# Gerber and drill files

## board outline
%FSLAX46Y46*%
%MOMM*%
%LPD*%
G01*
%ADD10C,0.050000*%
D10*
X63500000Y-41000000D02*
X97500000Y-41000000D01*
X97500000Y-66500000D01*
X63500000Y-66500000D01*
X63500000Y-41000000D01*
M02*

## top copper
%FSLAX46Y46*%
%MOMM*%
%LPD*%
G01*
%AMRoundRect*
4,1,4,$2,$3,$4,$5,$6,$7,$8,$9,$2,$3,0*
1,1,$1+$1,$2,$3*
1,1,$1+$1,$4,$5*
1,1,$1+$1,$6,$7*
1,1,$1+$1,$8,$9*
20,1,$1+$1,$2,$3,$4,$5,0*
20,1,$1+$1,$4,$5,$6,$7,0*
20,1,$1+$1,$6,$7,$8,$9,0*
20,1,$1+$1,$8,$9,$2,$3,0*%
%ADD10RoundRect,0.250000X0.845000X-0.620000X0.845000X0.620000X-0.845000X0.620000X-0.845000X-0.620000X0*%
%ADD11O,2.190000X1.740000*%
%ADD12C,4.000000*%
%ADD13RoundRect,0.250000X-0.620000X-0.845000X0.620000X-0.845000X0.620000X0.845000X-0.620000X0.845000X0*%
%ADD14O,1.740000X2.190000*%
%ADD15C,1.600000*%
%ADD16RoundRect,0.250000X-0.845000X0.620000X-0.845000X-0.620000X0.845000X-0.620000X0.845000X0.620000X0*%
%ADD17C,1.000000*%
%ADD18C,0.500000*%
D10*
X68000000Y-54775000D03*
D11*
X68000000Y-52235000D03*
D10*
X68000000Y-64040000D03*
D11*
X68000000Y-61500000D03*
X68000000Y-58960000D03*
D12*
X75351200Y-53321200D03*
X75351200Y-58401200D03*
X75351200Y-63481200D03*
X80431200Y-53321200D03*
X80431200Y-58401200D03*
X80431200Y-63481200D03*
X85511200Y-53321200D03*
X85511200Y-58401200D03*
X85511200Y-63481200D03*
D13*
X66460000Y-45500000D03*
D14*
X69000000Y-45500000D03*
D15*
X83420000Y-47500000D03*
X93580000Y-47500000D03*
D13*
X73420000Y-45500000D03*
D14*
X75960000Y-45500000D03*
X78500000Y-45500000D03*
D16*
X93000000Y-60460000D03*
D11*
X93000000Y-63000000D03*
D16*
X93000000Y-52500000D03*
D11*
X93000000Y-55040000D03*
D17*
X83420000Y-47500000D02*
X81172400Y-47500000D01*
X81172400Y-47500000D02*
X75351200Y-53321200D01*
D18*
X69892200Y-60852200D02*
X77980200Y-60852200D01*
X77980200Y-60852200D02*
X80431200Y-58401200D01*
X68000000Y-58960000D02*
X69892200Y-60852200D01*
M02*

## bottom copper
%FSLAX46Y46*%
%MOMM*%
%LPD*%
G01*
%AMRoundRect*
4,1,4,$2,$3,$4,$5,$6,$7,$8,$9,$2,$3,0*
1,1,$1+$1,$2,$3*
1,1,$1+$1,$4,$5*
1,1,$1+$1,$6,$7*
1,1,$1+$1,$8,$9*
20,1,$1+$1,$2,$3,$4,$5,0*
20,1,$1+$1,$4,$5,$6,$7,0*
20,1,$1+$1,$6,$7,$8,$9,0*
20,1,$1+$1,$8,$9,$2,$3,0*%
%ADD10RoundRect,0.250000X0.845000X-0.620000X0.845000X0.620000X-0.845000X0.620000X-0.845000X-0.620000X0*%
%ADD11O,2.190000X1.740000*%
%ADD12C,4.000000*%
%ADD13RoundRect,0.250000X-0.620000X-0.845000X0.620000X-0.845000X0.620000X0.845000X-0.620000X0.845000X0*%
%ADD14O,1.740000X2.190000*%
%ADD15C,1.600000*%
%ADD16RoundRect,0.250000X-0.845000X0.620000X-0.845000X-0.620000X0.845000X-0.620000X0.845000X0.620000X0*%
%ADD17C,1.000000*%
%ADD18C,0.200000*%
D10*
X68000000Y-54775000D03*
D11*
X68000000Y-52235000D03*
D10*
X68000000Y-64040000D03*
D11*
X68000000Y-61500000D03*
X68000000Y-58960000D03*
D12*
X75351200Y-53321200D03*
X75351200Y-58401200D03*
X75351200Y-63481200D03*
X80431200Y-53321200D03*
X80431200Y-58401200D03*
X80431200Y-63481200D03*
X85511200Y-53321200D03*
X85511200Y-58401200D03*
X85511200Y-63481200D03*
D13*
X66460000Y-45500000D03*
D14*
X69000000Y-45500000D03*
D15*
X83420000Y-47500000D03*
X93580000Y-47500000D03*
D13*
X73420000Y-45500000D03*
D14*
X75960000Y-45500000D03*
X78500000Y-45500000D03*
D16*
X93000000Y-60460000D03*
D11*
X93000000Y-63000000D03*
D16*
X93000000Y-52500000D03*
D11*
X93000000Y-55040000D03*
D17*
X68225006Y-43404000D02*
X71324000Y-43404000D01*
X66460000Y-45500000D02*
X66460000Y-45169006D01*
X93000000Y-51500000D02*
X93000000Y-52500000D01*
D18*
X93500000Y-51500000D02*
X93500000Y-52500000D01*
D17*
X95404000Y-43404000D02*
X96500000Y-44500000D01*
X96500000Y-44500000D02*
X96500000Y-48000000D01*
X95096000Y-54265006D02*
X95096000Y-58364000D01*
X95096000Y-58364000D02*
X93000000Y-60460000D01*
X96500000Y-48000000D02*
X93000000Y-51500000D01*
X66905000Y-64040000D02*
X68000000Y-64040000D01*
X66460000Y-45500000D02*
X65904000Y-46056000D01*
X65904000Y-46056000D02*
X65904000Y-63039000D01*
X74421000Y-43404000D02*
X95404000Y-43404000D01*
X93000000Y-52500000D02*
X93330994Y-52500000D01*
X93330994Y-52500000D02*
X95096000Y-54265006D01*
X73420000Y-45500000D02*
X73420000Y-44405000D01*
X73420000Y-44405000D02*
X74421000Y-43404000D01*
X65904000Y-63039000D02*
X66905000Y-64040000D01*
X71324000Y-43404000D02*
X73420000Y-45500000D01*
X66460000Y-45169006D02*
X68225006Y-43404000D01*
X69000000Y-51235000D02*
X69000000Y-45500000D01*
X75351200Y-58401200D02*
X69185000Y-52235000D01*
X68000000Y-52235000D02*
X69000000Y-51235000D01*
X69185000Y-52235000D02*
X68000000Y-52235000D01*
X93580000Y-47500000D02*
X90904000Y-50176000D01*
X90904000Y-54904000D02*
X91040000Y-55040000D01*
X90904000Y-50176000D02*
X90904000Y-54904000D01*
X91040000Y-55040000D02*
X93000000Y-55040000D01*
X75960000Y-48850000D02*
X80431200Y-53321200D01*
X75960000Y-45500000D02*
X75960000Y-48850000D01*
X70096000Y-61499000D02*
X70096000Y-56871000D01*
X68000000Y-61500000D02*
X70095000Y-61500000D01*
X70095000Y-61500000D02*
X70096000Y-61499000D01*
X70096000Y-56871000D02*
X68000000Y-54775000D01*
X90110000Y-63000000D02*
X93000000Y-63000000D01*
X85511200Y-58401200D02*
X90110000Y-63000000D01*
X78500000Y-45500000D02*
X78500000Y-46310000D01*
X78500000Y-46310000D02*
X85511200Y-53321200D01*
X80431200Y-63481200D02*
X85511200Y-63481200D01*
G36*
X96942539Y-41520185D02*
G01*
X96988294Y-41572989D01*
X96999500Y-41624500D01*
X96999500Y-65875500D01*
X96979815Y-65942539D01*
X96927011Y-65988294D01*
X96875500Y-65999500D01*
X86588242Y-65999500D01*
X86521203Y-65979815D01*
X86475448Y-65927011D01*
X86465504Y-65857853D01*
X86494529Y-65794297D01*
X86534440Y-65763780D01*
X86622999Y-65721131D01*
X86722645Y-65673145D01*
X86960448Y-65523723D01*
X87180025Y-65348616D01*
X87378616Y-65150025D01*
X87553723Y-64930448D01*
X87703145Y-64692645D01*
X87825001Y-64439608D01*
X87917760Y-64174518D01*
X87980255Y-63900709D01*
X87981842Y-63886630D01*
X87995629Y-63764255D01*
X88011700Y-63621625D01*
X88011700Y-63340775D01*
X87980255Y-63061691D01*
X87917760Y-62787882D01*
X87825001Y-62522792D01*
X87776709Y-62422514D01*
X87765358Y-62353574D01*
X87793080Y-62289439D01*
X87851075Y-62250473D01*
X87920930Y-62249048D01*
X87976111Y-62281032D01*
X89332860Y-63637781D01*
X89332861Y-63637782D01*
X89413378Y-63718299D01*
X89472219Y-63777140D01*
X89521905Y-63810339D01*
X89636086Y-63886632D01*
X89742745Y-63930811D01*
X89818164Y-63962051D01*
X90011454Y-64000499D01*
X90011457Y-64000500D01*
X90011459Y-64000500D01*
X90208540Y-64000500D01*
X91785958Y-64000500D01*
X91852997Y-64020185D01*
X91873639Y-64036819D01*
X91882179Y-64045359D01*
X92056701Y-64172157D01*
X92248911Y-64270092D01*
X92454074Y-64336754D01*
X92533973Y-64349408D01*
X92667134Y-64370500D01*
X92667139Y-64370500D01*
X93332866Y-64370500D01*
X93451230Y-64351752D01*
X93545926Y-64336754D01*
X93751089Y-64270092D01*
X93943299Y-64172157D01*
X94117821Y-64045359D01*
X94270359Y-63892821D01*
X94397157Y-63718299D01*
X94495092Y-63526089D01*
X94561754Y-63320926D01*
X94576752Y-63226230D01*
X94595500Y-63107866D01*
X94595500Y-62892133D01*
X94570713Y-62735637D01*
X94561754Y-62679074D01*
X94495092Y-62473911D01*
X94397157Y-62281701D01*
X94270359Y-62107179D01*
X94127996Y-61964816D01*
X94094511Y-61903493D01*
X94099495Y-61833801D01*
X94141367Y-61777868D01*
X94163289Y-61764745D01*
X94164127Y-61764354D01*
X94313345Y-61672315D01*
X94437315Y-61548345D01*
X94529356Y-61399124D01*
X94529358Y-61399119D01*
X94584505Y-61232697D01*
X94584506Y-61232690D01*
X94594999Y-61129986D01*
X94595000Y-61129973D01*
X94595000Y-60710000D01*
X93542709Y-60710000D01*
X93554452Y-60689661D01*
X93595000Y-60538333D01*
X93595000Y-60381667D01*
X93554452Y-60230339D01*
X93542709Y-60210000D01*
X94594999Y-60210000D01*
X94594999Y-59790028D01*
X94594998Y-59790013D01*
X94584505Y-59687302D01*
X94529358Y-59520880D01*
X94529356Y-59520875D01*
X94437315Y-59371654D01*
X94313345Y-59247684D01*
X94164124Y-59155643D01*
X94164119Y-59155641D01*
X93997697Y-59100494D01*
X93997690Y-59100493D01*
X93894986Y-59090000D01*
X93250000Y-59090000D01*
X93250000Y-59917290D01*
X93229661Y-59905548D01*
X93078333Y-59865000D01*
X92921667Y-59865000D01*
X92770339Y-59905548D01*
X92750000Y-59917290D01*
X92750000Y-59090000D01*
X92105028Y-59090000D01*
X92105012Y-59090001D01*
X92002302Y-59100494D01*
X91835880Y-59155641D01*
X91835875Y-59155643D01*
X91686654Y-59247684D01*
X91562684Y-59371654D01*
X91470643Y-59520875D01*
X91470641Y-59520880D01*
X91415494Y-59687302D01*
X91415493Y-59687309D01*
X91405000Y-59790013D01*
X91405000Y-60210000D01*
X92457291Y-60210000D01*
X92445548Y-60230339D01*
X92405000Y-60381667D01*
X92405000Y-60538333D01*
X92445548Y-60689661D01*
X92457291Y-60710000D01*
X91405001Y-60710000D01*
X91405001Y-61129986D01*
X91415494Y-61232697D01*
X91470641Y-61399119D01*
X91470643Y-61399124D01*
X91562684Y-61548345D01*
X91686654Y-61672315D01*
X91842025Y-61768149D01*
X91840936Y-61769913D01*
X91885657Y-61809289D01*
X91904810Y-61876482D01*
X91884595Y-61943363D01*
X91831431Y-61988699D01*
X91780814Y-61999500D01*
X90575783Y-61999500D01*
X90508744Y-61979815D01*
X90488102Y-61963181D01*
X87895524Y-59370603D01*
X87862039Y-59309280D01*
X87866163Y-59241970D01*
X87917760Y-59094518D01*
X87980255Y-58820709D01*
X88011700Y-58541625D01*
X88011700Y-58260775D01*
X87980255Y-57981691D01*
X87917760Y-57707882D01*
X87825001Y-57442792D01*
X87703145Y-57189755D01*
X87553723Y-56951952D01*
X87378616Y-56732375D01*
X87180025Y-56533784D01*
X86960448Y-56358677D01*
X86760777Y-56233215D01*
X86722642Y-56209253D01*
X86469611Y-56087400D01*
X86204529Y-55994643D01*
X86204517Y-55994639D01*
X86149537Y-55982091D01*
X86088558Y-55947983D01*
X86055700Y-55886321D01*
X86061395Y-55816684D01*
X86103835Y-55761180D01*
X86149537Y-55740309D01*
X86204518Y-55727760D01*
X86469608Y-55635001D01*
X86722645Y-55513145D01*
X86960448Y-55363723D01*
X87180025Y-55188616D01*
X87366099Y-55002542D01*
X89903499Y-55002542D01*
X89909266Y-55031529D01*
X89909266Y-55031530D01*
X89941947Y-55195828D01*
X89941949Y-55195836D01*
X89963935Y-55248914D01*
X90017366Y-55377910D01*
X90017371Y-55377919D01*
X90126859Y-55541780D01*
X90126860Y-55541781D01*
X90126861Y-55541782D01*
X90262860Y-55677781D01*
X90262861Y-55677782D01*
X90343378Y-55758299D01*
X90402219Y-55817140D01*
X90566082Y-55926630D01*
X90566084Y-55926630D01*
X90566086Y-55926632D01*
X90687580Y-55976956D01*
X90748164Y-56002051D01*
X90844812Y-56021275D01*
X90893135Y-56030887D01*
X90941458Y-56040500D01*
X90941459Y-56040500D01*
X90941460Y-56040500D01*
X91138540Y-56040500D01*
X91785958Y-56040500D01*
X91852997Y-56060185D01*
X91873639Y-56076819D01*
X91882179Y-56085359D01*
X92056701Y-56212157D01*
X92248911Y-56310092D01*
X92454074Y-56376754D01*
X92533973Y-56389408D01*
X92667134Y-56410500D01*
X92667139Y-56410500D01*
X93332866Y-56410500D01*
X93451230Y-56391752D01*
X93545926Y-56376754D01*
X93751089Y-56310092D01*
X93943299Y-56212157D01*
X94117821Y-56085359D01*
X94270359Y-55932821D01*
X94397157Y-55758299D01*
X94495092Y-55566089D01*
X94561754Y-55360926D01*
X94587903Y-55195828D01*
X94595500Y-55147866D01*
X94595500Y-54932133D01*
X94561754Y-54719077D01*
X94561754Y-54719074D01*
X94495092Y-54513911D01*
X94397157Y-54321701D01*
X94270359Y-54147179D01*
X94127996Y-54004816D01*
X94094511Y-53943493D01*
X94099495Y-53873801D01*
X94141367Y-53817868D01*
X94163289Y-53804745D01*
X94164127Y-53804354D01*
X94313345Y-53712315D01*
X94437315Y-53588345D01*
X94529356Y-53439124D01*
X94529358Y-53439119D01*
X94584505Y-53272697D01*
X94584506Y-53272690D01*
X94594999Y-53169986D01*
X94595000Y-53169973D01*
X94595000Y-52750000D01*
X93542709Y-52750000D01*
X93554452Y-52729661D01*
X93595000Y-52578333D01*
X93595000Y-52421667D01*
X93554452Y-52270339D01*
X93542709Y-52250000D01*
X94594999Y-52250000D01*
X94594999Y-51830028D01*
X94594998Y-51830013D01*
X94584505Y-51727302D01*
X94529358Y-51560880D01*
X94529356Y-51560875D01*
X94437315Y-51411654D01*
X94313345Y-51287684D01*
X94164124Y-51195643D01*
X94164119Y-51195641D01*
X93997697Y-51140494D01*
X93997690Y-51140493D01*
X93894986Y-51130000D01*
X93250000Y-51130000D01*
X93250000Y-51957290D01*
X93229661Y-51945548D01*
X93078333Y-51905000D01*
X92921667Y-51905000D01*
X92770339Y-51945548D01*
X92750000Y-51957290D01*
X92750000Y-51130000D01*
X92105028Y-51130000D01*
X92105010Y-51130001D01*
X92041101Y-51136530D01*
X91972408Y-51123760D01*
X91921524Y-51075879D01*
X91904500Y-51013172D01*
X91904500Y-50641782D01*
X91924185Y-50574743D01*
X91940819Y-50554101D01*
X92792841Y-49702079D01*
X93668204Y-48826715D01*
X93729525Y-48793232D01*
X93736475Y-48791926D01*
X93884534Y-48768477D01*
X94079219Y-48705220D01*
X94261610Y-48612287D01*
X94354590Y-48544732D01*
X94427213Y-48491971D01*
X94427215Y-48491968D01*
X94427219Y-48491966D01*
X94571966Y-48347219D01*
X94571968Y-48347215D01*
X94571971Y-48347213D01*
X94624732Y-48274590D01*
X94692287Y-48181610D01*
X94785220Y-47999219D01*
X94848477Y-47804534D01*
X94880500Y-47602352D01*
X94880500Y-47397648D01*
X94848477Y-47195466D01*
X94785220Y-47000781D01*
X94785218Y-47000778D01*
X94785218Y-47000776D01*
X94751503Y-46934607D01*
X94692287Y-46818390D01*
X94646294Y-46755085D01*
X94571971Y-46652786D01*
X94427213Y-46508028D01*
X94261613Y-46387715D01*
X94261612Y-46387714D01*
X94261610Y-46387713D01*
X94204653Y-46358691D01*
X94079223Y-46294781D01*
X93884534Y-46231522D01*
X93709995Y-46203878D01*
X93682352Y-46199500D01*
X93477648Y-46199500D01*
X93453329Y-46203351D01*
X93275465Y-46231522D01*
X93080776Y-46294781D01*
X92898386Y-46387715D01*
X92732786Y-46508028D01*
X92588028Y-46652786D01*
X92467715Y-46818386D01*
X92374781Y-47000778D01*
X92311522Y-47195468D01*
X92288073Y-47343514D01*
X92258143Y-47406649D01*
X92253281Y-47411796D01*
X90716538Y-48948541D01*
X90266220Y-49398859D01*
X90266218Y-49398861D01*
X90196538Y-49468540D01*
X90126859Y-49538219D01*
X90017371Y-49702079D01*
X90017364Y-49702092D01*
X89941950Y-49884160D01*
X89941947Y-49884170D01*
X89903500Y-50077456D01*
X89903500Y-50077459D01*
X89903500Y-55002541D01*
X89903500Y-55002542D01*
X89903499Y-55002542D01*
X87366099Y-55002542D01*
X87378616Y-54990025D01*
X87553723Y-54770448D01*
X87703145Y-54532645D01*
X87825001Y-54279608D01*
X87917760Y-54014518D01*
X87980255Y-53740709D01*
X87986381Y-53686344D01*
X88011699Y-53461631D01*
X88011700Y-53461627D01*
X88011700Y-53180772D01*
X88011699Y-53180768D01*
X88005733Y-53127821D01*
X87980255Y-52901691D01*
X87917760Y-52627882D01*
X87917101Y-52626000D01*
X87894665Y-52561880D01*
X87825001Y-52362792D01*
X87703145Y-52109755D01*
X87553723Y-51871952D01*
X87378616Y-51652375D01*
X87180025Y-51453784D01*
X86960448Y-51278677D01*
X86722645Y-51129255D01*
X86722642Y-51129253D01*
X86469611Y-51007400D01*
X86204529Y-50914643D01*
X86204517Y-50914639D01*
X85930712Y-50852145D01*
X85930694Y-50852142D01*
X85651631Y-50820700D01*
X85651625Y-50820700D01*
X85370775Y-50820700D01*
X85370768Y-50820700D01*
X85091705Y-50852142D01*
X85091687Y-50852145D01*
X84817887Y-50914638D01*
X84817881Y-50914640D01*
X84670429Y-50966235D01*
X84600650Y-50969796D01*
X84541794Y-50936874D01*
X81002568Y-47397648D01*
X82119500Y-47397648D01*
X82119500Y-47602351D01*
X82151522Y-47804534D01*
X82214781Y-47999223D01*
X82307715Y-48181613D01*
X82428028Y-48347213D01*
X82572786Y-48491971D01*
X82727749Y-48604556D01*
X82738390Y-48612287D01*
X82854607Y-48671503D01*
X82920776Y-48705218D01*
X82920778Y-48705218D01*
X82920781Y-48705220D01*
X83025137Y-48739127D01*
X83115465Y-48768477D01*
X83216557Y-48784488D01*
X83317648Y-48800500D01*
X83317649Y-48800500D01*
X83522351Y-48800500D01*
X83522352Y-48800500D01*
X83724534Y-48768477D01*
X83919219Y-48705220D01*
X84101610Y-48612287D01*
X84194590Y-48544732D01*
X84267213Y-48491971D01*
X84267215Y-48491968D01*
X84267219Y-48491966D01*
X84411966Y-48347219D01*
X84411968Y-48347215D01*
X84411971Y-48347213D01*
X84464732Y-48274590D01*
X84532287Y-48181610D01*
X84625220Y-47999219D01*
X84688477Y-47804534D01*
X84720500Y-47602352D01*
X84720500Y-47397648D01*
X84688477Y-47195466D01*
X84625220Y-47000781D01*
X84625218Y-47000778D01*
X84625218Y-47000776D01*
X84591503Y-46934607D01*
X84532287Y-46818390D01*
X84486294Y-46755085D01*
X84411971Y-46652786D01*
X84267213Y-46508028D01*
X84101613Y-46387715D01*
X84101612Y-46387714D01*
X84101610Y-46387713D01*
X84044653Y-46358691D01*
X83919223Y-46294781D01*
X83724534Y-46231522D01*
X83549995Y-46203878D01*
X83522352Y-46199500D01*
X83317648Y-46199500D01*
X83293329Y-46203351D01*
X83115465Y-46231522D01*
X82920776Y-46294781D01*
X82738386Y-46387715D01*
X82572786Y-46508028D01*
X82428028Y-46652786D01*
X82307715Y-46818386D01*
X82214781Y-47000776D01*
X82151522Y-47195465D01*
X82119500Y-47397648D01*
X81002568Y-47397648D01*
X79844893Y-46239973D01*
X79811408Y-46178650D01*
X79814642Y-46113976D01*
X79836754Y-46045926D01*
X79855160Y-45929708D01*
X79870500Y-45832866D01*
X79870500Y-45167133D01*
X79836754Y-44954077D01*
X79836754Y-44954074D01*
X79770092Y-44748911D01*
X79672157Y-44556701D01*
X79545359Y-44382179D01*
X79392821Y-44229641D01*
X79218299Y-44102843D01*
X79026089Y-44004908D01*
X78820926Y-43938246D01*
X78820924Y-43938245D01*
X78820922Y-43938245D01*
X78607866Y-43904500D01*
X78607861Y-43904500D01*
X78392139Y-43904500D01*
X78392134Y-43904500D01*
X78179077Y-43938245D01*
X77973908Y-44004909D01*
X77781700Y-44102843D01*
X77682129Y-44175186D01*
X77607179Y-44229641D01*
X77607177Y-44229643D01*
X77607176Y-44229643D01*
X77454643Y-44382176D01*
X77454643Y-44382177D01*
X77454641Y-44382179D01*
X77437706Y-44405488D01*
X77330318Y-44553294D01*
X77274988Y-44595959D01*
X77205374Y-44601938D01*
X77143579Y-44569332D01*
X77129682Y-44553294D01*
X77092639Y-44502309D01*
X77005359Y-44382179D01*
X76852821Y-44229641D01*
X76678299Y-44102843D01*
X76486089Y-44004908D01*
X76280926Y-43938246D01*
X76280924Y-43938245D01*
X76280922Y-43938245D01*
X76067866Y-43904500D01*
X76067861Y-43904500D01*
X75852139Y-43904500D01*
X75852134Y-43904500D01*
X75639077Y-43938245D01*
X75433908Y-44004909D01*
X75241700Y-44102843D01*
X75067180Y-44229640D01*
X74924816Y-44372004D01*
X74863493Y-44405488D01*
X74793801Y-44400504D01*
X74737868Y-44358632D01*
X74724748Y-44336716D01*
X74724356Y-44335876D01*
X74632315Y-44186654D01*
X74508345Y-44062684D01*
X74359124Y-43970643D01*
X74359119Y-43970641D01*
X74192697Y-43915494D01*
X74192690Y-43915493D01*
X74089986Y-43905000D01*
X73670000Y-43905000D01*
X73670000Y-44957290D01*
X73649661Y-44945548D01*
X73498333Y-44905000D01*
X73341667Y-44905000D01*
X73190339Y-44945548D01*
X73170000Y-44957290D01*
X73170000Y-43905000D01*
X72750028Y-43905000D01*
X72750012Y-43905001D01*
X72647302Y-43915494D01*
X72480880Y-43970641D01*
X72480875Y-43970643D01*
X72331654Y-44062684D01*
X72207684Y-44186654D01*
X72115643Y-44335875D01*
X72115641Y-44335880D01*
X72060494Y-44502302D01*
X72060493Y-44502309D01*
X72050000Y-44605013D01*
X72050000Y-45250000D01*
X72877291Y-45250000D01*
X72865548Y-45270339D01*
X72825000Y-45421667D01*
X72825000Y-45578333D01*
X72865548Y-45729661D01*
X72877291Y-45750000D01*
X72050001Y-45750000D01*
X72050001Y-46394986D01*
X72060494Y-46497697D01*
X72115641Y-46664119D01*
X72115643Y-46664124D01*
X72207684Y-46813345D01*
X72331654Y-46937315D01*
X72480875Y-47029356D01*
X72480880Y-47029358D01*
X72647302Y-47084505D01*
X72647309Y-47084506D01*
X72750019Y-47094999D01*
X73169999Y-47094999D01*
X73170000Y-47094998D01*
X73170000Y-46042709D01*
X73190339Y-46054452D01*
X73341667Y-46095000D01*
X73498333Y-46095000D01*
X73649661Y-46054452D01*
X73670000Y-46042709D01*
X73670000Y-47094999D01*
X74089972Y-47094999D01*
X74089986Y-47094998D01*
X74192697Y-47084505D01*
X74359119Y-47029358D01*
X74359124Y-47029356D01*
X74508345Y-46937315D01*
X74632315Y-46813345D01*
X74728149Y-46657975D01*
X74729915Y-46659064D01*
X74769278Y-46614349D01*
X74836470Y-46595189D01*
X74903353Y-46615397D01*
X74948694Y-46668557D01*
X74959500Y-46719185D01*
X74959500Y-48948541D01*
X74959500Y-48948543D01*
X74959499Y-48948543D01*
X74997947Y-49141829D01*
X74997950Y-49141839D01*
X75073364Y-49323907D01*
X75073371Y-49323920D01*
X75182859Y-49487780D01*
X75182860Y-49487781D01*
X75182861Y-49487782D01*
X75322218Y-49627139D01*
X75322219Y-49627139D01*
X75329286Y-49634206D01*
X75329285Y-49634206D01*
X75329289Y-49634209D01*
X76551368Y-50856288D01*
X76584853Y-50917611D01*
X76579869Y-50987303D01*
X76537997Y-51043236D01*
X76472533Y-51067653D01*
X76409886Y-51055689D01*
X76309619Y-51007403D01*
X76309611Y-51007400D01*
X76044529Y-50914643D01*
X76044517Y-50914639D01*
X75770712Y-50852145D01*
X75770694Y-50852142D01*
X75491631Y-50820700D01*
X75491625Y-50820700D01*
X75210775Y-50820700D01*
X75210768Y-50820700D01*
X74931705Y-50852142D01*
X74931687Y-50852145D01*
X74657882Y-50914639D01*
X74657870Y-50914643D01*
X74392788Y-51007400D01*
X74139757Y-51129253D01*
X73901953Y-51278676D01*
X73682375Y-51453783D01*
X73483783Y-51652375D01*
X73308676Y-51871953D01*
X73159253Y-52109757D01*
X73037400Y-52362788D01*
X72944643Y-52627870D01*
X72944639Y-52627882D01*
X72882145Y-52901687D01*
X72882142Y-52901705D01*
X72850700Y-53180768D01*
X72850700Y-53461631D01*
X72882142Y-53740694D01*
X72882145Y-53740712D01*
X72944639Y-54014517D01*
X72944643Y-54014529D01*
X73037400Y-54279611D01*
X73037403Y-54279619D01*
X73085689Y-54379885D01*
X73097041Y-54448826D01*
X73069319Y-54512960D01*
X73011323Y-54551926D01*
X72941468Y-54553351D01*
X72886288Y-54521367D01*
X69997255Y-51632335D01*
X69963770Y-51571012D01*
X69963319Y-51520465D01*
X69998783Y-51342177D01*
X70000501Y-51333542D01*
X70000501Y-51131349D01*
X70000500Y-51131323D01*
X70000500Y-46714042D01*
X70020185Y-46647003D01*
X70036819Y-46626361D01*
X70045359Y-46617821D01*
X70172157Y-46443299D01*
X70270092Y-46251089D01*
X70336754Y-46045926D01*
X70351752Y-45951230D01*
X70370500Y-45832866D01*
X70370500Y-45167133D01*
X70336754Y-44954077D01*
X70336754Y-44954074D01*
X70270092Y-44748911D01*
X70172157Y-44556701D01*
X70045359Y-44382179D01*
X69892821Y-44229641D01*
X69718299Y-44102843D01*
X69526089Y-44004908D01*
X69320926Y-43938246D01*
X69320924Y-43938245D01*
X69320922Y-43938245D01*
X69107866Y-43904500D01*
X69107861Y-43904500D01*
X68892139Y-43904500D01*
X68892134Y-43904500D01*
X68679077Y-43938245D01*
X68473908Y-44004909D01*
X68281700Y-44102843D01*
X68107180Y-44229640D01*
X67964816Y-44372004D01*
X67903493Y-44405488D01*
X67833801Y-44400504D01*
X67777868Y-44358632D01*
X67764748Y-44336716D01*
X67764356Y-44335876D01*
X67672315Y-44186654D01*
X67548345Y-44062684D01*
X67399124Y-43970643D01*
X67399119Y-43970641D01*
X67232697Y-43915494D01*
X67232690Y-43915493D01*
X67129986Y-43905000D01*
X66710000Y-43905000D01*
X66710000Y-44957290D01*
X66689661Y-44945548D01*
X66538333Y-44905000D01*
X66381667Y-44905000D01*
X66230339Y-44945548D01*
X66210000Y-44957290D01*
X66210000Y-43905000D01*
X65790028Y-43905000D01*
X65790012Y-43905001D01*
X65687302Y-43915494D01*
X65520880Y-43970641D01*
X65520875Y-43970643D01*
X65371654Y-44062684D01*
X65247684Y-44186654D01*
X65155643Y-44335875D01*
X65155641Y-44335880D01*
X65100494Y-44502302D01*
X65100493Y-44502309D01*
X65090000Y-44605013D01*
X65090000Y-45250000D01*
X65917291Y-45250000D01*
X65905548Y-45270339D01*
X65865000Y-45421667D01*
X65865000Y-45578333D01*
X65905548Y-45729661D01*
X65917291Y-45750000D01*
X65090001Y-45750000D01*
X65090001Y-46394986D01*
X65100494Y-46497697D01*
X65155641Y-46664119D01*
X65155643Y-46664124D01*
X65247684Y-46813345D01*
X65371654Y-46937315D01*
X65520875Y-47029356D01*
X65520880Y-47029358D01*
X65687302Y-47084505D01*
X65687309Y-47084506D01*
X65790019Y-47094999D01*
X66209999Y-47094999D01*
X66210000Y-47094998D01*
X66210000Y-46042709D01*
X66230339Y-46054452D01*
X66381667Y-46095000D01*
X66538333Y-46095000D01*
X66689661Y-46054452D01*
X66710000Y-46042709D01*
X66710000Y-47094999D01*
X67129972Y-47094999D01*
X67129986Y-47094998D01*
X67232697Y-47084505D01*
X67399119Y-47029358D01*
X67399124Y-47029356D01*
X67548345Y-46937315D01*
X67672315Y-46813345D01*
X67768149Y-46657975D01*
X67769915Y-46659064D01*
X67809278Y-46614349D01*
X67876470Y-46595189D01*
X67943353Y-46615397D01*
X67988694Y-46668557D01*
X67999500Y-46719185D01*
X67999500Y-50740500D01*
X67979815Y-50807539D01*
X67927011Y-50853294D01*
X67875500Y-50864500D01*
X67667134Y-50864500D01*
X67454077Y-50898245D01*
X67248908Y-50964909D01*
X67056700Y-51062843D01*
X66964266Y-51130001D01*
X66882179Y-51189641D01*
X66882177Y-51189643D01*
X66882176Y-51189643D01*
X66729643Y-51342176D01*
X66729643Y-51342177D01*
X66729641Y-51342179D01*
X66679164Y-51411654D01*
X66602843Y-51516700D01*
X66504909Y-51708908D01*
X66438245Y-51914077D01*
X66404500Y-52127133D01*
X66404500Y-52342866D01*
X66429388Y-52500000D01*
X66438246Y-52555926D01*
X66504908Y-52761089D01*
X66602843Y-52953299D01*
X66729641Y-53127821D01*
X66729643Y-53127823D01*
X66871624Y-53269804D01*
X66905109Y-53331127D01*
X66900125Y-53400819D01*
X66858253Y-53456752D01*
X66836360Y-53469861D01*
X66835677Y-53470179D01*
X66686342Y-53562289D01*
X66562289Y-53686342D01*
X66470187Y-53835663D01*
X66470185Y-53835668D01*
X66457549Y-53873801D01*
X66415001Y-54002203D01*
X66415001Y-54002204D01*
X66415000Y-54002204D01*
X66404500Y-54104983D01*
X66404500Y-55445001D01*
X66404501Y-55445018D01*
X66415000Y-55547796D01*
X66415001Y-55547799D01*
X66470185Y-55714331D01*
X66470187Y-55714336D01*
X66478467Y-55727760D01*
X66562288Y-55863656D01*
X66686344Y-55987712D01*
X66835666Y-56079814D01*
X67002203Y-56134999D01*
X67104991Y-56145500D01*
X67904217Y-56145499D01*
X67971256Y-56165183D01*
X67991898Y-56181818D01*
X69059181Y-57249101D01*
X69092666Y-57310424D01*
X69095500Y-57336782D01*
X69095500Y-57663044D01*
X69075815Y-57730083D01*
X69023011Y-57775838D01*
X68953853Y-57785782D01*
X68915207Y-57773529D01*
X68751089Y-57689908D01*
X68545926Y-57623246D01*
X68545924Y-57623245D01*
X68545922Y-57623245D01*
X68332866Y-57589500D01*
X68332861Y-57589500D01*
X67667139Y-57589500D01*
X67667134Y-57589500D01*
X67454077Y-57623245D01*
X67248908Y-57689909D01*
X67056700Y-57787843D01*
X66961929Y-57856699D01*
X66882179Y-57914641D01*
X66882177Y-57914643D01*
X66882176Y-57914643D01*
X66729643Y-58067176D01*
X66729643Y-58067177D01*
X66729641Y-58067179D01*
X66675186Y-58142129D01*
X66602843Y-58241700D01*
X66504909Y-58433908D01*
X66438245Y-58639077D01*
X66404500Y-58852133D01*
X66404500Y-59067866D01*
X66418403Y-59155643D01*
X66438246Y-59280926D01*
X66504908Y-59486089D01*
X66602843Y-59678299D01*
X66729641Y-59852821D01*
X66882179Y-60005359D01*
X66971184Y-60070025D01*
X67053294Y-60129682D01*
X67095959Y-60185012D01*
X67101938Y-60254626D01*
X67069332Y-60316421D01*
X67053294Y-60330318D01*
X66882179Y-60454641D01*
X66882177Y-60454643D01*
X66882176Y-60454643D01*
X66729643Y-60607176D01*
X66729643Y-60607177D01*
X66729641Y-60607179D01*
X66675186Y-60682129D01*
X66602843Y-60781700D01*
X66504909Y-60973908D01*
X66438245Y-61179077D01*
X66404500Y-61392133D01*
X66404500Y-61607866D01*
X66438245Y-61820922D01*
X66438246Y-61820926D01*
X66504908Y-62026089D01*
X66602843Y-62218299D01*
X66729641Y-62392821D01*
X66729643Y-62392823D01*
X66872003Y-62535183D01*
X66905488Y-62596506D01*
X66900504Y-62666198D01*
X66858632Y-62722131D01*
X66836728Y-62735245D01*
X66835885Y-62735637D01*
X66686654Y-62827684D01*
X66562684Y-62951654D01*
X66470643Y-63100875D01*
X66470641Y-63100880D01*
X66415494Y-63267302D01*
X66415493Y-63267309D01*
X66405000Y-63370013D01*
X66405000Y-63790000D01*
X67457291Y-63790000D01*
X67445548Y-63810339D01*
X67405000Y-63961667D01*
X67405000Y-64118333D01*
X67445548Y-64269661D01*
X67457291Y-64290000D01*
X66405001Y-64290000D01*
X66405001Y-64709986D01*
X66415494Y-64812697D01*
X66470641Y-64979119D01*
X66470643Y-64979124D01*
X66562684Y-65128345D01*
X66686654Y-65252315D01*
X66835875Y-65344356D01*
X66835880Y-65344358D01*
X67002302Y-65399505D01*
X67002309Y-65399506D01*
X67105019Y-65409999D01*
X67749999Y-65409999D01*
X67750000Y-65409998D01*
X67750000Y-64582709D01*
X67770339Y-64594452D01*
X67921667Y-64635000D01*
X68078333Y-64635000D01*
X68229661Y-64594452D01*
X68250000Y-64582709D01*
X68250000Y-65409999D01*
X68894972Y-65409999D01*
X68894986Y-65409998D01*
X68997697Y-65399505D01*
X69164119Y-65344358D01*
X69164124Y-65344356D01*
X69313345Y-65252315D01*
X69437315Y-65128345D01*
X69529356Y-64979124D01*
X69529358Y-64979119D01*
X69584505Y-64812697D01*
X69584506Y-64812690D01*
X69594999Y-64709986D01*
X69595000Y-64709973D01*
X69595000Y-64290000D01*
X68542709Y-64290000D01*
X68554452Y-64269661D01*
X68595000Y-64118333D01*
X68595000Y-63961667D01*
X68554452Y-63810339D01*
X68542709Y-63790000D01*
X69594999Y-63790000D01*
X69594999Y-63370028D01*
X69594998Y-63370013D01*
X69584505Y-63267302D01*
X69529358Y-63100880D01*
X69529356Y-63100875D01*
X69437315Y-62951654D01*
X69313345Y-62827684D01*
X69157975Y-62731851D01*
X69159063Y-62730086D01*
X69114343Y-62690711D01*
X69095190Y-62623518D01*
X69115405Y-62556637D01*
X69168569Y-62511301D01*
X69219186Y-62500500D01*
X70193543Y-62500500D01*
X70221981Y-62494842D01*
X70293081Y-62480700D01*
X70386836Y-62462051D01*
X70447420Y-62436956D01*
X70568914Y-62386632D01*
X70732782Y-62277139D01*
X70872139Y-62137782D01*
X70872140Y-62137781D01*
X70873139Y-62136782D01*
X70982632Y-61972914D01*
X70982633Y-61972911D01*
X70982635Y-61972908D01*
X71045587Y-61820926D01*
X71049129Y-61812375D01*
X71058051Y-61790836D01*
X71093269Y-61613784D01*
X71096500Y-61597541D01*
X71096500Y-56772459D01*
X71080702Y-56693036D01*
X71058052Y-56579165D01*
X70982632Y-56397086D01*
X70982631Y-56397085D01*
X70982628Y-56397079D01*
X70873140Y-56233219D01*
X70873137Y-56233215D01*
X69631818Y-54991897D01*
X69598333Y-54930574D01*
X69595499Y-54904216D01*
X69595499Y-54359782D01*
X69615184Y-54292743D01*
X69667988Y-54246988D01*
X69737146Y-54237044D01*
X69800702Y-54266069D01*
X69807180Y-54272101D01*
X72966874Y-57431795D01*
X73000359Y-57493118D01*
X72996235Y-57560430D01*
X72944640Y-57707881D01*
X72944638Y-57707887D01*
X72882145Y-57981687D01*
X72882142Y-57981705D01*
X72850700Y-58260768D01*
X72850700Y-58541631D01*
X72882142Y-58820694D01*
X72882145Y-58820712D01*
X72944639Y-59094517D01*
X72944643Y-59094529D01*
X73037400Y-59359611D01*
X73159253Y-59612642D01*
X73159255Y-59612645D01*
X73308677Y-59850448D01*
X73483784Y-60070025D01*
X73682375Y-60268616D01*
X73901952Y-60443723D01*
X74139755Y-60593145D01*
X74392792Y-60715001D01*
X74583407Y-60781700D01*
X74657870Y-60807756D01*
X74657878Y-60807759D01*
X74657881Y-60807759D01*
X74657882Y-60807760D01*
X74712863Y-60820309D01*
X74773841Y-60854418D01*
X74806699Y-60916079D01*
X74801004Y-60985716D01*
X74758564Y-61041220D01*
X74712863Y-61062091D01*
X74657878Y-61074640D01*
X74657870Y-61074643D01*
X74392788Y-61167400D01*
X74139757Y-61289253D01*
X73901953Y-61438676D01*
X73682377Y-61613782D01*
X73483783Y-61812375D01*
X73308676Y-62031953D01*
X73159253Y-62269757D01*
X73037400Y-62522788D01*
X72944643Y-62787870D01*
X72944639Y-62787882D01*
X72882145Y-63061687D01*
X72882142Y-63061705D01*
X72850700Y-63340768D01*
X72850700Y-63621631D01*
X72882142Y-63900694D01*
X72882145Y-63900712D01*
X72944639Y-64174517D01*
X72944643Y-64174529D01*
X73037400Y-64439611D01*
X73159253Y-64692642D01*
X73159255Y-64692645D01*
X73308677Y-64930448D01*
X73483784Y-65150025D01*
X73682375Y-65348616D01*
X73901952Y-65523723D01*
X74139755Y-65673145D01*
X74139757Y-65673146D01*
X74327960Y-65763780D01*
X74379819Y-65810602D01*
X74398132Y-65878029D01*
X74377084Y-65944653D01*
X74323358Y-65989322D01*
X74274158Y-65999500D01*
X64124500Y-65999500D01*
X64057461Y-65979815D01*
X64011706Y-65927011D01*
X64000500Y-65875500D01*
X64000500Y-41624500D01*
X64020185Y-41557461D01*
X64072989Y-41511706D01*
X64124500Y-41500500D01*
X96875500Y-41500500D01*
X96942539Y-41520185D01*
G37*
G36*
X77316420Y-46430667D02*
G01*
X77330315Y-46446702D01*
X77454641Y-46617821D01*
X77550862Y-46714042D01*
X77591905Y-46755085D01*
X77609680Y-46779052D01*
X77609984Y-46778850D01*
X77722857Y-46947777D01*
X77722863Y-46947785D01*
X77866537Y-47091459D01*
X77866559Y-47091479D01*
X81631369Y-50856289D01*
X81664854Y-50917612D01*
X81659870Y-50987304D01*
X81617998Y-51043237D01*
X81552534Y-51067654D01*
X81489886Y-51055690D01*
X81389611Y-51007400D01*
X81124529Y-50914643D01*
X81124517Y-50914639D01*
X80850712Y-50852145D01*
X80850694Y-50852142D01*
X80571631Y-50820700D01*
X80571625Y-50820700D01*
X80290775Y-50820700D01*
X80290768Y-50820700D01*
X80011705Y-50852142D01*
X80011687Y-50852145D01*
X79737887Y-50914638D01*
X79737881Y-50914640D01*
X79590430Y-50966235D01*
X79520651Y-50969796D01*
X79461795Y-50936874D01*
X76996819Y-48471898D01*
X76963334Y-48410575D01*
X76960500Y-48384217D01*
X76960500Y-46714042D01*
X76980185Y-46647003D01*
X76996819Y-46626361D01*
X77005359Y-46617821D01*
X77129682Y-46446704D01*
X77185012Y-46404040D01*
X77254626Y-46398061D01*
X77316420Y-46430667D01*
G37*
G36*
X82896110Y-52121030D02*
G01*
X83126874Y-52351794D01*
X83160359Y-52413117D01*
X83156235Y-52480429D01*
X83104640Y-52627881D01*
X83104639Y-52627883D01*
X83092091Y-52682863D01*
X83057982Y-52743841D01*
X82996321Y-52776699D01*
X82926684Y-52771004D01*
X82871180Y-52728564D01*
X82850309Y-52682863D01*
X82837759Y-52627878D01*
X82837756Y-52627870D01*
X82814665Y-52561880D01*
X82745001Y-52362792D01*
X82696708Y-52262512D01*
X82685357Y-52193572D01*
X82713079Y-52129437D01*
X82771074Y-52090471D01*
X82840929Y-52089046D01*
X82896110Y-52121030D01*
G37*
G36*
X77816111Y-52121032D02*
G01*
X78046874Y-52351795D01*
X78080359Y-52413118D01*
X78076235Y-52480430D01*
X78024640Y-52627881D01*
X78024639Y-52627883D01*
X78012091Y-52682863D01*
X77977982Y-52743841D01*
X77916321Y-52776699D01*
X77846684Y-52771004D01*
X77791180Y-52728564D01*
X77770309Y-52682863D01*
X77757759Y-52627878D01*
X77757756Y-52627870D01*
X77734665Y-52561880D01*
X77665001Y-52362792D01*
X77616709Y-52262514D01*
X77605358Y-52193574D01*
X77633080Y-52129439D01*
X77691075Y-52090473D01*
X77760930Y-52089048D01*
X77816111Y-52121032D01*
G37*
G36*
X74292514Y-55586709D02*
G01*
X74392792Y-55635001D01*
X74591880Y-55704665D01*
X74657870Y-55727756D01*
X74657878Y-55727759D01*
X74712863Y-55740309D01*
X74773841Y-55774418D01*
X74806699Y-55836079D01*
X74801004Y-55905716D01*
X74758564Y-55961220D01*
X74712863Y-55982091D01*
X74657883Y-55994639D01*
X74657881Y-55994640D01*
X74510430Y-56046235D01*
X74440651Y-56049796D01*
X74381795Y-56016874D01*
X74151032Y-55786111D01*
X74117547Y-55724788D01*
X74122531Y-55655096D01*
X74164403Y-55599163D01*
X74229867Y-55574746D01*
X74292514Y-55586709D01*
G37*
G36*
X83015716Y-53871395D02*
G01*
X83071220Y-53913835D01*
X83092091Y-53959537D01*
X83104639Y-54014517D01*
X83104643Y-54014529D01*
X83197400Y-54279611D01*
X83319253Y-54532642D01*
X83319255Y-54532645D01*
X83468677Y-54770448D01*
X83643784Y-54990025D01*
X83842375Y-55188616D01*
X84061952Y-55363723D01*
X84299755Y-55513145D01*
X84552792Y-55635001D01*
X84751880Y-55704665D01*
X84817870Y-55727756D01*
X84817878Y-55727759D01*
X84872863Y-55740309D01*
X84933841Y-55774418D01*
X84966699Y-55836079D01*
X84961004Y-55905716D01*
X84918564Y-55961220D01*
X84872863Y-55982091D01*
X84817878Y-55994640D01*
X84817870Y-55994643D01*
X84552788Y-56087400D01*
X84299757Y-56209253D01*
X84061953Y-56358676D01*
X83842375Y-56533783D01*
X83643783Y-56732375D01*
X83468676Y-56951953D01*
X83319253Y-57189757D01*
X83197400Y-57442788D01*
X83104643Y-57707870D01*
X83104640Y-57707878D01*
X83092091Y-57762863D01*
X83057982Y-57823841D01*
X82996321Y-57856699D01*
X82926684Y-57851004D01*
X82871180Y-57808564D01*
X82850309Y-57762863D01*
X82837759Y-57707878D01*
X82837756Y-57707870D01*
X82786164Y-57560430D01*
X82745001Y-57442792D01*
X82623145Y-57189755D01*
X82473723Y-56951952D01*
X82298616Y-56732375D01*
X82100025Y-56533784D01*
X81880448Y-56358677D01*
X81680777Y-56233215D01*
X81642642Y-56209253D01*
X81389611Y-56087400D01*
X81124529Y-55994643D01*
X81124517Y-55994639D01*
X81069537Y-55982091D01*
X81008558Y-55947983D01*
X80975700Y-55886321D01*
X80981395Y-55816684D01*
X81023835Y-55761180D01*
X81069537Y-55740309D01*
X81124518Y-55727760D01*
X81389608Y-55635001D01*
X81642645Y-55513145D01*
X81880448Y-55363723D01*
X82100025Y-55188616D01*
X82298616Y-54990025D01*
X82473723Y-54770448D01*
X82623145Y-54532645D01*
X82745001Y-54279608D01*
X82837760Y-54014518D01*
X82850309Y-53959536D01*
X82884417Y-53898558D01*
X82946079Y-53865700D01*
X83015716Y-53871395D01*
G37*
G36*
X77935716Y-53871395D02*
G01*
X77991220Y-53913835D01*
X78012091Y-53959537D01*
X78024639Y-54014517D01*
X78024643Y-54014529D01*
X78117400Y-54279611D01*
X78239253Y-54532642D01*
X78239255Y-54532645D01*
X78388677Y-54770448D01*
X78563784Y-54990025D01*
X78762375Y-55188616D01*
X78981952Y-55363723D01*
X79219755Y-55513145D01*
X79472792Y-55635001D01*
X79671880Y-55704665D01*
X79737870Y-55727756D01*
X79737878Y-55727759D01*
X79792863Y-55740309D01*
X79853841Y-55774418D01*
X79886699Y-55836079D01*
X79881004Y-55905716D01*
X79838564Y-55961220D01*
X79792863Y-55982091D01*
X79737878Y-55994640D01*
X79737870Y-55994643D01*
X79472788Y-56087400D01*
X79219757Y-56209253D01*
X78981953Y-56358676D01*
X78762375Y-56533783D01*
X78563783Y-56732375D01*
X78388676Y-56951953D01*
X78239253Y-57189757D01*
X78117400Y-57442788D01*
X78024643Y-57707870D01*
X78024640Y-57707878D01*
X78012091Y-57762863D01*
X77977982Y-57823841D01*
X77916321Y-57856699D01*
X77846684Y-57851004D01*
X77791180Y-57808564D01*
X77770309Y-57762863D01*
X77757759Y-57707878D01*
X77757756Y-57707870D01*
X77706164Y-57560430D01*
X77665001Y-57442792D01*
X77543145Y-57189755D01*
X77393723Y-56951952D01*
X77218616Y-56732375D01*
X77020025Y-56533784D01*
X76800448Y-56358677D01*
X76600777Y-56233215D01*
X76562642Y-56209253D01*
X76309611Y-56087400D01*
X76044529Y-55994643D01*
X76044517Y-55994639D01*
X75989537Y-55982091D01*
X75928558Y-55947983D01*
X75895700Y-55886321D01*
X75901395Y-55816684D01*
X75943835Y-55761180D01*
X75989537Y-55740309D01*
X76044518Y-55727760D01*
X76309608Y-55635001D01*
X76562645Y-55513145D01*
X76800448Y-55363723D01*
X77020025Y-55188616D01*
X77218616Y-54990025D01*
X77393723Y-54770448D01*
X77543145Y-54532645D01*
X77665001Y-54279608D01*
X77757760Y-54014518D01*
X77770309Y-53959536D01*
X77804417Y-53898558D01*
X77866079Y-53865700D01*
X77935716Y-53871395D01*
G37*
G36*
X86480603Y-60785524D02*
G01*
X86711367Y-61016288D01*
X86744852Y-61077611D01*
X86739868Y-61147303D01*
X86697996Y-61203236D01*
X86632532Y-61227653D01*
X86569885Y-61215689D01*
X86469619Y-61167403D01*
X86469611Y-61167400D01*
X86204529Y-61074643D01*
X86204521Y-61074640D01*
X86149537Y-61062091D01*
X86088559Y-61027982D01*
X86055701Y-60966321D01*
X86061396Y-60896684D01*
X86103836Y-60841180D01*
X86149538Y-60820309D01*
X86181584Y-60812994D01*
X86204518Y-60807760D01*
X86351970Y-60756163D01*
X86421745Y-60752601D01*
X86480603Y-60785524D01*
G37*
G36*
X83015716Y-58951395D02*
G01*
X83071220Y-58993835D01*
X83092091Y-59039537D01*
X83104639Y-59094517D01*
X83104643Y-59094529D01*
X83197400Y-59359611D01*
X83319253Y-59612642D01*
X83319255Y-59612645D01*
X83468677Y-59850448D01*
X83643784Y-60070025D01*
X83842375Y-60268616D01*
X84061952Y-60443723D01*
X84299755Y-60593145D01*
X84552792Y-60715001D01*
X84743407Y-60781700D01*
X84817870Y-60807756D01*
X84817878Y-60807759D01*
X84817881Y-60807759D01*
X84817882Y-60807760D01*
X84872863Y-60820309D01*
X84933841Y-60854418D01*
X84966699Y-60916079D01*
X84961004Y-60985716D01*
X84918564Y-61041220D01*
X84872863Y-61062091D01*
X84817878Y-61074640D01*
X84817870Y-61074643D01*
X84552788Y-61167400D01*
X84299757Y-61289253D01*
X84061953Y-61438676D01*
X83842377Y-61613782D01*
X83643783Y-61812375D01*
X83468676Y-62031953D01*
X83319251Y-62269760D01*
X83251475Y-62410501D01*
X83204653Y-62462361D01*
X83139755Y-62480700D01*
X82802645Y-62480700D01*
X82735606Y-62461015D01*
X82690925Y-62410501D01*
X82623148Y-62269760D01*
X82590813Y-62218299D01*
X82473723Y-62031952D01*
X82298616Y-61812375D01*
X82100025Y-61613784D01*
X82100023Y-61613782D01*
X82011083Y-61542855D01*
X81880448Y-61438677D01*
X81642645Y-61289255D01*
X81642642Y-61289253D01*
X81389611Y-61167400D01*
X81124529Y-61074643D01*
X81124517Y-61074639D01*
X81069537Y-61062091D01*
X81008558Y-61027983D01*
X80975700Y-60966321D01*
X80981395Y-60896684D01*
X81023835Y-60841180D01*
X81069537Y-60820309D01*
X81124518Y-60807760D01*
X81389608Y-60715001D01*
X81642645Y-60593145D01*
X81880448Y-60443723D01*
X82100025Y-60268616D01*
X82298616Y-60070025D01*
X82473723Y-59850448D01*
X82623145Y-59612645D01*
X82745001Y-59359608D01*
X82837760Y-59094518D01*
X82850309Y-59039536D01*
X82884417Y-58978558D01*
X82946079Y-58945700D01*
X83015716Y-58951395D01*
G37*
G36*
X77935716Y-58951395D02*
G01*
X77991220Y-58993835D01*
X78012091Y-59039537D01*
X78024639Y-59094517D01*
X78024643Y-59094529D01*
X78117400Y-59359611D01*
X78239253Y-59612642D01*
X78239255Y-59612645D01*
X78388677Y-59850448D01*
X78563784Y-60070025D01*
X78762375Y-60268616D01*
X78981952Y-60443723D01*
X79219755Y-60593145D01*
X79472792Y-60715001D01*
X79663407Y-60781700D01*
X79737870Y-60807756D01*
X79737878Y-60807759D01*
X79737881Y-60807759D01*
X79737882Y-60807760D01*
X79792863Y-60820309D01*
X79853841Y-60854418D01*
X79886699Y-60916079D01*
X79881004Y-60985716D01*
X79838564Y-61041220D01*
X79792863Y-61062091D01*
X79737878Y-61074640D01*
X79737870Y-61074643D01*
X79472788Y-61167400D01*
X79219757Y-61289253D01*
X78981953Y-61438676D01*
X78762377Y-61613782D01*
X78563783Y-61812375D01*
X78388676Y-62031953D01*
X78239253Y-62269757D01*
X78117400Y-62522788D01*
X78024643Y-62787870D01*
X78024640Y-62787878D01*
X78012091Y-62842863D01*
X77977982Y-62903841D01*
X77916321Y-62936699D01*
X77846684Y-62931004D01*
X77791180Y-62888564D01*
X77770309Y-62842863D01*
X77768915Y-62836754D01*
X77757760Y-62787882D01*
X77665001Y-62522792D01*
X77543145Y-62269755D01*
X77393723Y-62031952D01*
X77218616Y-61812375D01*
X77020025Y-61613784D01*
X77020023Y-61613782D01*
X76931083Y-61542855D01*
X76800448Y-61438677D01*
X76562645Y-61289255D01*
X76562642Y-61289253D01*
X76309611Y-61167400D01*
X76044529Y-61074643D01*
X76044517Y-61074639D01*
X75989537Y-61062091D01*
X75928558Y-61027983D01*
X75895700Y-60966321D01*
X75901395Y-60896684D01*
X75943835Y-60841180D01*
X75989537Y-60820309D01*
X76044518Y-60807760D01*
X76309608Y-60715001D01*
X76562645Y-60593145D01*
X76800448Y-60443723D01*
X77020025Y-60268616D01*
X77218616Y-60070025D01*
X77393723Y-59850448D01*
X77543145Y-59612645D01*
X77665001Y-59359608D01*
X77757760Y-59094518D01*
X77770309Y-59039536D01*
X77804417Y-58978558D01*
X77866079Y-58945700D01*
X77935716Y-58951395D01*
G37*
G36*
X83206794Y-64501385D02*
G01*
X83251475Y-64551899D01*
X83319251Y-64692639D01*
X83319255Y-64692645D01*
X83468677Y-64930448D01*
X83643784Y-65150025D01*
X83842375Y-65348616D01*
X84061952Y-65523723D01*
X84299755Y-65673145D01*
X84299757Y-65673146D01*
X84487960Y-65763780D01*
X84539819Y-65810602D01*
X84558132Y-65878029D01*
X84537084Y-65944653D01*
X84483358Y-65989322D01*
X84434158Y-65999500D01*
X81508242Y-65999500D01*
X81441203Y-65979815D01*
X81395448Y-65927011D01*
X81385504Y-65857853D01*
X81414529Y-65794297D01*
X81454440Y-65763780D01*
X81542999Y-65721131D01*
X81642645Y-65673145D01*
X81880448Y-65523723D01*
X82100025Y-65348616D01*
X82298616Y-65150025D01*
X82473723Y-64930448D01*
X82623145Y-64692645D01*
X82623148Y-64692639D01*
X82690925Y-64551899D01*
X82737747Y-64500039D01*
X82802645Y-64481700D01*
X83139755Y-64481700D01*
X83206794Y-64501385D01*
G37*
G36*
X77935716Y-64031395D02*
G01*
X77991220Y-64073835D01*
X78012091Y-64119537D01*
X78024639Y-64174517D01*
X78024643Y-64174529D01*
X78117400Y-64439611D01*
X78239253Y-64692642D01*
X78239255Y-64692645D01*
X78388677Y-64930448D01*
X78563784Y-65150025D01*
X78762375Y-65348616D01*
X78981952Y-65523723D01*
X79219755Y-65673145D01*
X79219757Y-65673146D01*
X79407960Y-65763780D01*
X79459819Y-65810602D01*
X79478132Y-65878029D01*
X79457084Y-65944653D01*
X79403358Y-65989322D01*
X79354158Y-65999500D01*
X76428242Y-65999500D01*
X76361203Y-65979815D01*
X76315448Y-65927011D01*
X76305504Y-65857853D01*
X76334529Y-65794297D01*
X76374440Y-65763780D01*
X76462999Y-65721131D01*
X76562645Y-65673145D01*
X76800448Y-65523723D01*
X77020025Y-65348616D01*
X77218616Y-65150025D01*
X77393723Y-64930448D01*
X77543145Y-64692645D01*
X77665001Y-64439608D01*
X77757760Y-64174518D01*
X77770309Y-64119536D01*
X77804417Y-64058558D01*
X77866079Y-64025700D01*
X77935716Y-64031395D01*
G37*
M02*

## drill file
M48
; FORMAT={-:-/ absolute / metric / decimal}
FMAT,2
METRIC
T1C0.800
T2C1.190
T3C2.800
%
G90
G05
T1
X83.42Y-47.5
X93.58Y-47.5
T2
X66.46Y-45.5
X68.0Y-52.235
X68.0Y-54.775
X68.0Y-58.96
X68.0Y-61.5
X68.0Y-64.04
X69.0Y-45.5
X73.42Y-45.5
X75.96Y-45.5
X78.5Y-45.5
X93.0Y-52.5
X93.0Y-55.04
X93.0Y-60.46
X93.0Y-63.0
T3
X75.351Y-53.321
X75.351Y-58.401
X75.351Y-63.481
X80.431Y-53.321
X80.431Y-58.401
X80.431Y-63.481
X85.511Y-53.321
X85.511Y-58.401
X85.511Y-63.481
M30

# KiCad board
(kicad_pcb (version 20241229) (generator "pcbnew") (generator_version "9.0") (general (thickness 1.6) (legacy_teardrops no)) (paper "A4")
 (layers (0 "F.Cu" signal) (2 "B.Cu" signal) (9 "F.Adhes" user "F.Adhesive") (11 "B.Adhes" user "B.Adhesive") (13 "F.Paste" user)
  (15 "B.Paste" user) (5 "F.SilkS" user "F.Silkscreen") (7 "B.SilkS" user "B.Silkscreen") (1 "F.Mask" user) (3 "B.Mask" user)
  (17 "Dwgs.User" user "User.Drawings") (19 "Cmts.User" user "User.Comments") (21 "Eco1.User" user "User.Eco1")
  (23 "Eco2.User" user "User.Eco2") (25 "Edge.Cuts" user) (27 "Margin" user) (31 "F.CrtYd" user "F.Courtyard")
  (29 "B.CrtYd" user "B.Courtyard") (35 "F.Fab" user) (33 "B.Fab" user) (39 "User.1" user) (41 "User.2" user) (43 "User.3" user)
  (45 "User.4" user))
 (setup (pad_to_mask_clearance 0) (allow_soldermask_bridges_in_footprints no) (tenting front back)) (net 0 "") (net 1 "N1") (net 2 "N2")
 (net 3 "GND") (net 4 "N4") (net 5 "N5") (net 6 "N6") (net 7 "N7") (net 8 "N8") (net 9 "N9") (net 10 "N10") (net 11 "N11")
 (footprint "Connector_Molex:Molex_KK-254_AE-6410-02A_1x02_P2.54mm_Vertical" (layer "F.Cu") (at 68 54.775 90)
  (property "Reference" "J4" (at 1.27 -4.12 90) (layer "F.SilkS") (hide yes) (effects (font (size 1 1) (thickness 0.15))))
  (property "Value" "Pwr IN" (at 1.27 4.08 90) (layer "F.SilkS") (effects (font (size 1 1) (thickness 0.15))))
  (pad "1" thru_hole roundrect (at 0 0 90) (size 1.74 2.19) (drill 1.19) (layers "*.Cu" "*.Mask") (remove_unused_layers no)
   (roundrect_rratio 0.143678) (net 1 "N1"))
  (pad "2" thru_hole oval (at 2.54 0 90) (size 1.74 2.19) (drill 1.19) (layers "*.Cu" "*.Mask") (remove_unused_layers no) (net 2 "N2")))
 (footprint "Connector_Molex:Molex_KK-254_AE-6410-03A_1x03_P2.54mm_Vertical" (layer "F.Cu") (at 68 64.04 90)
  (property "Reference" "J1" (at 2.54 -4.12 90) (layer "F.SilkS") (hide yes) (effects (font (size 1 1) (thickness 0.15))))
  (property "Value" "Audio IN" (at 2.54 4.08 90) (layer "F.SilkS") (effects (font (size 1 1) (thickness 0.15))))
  (pad "1" thru_hole roundrect (at 0 0 90) (size 1.74 2.19) (drill 1.19) (layers "*.Cu" "*.Mask") (remove_unused_layers no)
   (roundrect_rratio 0.143678) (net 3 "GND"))
  (pad "2" thru_hole oval (at 2.54 0 90) (size 1.74 2.19) (drill 1.19) (layers "*.Cu" "*.Mask") (remove_unused_layers no) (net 1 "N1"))
  (pad "3" thru_hole oval (at 5.08 0 90) (size 1.74 2.19) (drill 1.19) (layers "*.Cu" "*.Mask") (remove_unused_layers no) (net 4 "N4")))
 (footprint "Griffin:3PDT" (layer "F.Cu") (at 80.4312 58.4012)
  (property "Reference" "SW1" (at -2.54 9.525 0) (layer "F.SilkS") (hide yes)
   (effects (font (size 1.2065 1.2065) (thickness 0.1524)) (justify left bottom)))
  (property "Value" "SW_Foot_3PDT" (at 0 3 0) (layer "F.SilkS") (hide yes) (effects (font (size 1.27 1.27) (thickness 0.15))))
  (pad "A1" thru_hole circle (at -5.08 -5.08 180) (size 4 4) (drill 2.8) (layers "*.Cu" "*.Mask") (remove_unused_layers no) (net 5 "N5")
   (solder_mask_margin 0.1016))
  (pad "A2" thru_hole circle (at -5.08 0 180) (size 4 4) (drill 2.8) (layers "*.Cu" "*.Mask") (remove_unused_layers no) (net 2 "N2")
   (solder_mask_margin 0.1016))
  (pad "A3" thru_hole circle (at -5.08 5.08 180) (size 4 4) (drill 2.8) (layers "*.Cu" "*.Mask") (remove_unused_layers no) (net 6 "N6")
   (solder_mask_margin 0.1016))
  (pad "B1" thru_hole circle (at 0 -5.08 180) (size 4 4) (drill 2.8) (layers "*.Cu" "*.Mask") (remove_unused_layers no) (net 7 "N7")
   (solder_mask_margin 0.1016))
  (pad "B2" thru_hole circle (at 0 0 180) (size 4 4) (drill 2.8) (layers "*.Cu" "*.Mask") (remove_unused_layers no) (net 4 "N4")
   (solder_mask_margin 0.1016))
  (pad "B3" thru_hole circle (at 0 5.08 180) (size 4 4) (drill 2.8) (layers "*.Cu" "*.Mask") (remove_unused_layers no) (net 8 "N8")
   (solder_mask_margin 0.1016))
  (pad "C1" thru_hole circle (at 5.08 -5.08 180) (size 4 4) (drill 2.8) (layers "*.Cu" "*.Mask") (remove_unused_layers no) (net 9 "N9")
   (solder_mask_margin 0.1016))
  (pad "C2" thru_hole circle (at 5.08 0 180) (size 4 4) (drill 2.8) (layers "*.Cu" "*.Mask") (remove_unused_layers no) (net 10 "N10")
   (solder_mask_margin 0.1016))
  (pad "C3" thru_hole circle (at 5.08 5.08 180) (size 4 4) (drill 2.8) (layers "*.Cu" "*.Mask") (remove_unused_layers no) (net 8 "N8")
   (solder_mask_margin 0.1016)))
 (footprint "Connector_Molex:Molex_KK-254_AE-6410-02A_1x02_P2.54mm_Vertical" (layer "F.Cu") (at 66.46 45.5)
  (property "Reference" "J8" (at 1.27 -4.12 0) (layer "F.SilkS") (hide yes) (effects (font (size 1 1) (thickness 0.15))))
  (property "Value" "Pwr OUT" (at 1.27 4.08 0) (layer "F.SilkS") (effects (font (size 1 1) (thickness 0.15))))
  (pad "1" thru_hole roundrect (at 0 0) (size 1.74 2.19) (drill 1.19) (layers "*.Cu" "*.Mask") (remove_unused_layers no)
   (roundrect_rratio 0.143678) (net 3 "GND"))
  (pad "2" thru_hole oval (at 2.54 0) (size 1.74 2.19) (drill 1.19) (layers "*.Cu" "*.Mask") (remove_unused_layers no) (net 2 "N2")))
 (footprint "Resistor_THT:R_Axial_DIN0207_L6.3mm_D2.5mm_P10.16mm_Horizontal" (layer "F.Cu") (at 83.42 47.5)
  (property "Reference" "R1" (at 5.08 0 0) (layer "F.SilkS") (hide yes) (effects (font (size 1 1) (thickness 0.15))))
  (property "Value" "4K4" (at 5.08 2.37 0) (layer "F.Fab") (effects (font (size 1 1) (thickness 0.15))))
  (pad "1" thru_hole circle (at 0 0) (size 1.6 1.6) (drill 0.8) (layers "*.Cu" "*.Mask") (remove_unused_layers no) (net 5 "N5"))
  (pad "2" thru_hole circle (at 10.16 0) (size 1.6 1.6) (drill 0.8) (layers "*.Cu" "*.Mask") (remove_unused_layers no) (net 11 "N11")))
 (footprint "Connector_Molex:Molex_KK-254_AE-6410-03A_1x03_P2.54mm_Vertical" (layer "F.Cu") (at 73.42 45.5)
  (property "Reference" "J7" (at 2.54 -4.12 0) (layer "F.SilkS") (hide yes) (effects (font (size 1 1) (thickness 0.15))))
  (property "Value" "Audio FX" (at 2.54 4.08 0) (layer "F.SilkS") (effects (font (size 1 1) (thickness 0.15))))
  (pad "1" thru_hole roundrect (at 0 0) (size 1.74 2.19) (drill 1.19) (layers "*.Cu" "*.Mask") (remove_unused_layers no)
   (roundrect_rratio 0.143678) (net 3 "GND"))
  (pad "2" thru_hole oval (at 2.54 0) (size 1.74 2.19) (drill 1.19) (layers "*.Cu" "*.Mask") (remove_unused_layers no) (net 7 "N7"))
  (pad "3" thru_hole oval (at 5.08 0) (size 1.74 2.19) (drill 1.19) (layers "*.Cu" "*.Mask") (remove_unused_layers no) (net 9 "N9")))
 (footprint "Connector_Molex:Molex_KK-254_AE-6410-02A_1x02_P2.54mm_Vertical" (layer "F.Cu") (at 93 60.46 -90)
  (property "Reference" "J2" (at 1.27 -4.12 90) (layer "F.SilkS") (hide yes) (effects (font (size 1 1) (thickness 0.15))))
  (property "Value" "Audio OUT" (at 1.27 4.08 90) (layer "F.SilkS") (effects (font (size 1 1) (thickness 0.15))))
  (pad "1" thru_hole roundrect (at 0 0 270) (size 1.74 2.19) (drill 1.19) (layers "*.Cu" "*.Mask") (remove_unused_layers no)
   (roundrect_rratio 0.143678) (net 3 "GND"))
  (pad "2" thru_hole oval (at 2.54 0 270) (size 1.74 2.19) (drill 1.19) (layers "*.Cu" "*.Mask") (remove_unused_layers no) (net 10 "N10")))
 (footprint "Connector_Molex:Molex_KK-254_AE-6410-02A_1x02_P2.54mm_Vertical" (layer "F.Cu") (at 93 52.5 -90)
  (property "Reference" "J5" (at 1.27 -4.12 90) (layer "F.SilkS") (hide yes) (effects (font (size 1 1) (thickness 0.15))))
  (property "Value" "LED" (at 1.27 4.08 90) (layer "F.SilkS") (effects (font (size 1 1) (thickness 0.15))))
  (pad "1" thru_hole roundrect (at 0 0 270) (size 1.74 2.19) (drill 1.19) (layers "*.Cu" "*.Mask") (remove_unused_layers no)
   (roundrect_rratio 0.143678) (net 3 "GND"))
  (pad "2" thru_hole oval (at 2.54 0 270) (size 1.74 2.19) (drill 1.19) (layers "*.Cu" "*.Mask") (remove_unused_layers no) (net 11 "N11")))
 (gr_rect (start 63.5 41) (end 97.5 66.5) (stroke (width 0.05) (type default)) (fill no) (layer "Edge.Cuts"))
 (segment (start 68.225006 43.404) (end 71.324 43.404) (width 1) (layer "B.Cu") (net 3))
 (segment (start 66.46 45.5) (end 66.46 45.169006) (width 1) (layer "B.Cu") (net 3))
 (segment (start 93 51.5) (end 93 52.5) (width 1) (layer "B.Cu") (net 3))
 (segment (start 93.5 51.5) (end 93.5 52.5) (width 0.2) (layer "B.Cu") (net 3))
 (segment (start 95.404 43.404) (end 96.5 44.5) (width 1) (layer "B.Cu") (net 3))
 (segment (start 96.5 44.5) (end 96.5 48) (width 1) (layer "B.Cu") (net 3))
 (segment (start 95.096 54.265006) (end 95.096 58.364) (width 1) (layer "B.Cu") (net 3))
 (segment (start 95.096 58.364) (end 93 60.46) (width 1) (layer "B.Cu") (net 3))
 (segment (start 96.5 48) (end 93 51.5) (width 1) (layer "B.Cu") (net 3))
 (segment (start 66.905 64.04) (end 68 64.04) (width 1) (layer "B.Cu") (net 3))
 (segment (start 66.46 45.5) (end 65.904 46.056) (width 1) (layer "B.Cu") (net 3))
 (segment (start 65.904 46.056) (end 65.904 63.039) (width 1) (layer "B.Cu") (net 3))
 (segment (start 74.421 43.404) (end 95.404 43.404) (width 1) (layer "B.Cu") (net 3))
 (segment (start 93 52.5) (end 93.330994 52.5) (width 1) (layer "B.Cu") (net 3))
 (segment (start 93.330994 52.5) (end 95.096 54.265006) (width 1) (layer "B.Cu") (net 3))
 (segment (start 73.42 45.5) (end 73.42 44.405) (width 1) (layer "B.Cu") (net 3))
 (segment (start 73.42 44.405) (end 74.421 43.404) (width 1) (layer "B.Cu") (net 3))
 (segment (start 65.904 63.039) (end 66.905 64.04) (width 1) (layer "B.Cu") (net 3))
 (segment (start 71.324 43.404) (end 73.42 45.5) (width 1) (layer "B.Cu") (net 3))
 (segment (start 66.46 45.169006) (end 68.225006 43.404) (width 1) (layer "B.Cu") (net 3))
 (segment (start 69 51.235) (end 69 45.5) (width 1) (layer "B.Cu") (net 2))
 (segment (start 75.3512 58.4012) (end 69.185 52.235) (width 1) (layer "B.Cu") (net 2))
 (segment (start 68 52.235) (end 69 51.235) (width 1) (layer "B.Cu") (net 2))
 (segment (start 69.185 52.235) (end 68 52.235) (width 1) (layer "B.Cu") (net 2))
 (segment (start 93.58 47.5) (end 90.904 50.176) (width 1) (layer "B.Cu") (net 11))
 (segment (start 90.904 54.904) (end 91.04 55.04) (width 1) (layer "B.Cu") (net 11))
 (segment (start 90.904 50.176) (end 90.904 54.904) (width 1) (layer "B.Cu") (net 11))
 (segment (start 91.04 55.04) (end 93 55.04) (width 1) (layer "B.Cu") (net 11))
 (segment (start 75.96 48.85) (end 80.4312 53.3212) (width 1) (layer "B.Cu") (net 7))
 (segment (start 75.96 45.5) (end 75.96 48.85) (width 1) (layer "B.Cu") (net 7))
 (segment (start 83.42 47.5) (end 81.1724 47.5) (width 1) (layer "F.Cu") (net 5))
 (segment (start 81.1724 47.5) (end 75.3512 53.3212) (width 1) (layer "F.Cu") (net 5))
 (segment (start 69.8922 60.8522) (end 77.9802 60.8522) (width 0.5) (layer "F.Cu") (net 4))
 (segment (start 77.9802 60.8522) (end 80.4312 58.4012) (width 0.5) (layer "F.Cu") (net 4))
 (segment (start 68 58.96) (end 69.8922 60.8522) (width 0.5) (layer "F.Cu") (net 4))
 (segment (start 70.096 61.499) (end 70.096 56.871) (width 1) (layer "B.Cu") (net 1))
 (segment (start 68 61.5) (end 70.095 61.5) (width 1) (layer "B.Cu") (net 1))
 (segment (start 70.095 61.5) (end 70.096 61.499) (width 1) (layer "B.Cu") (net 1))
 (segment (start 70.096 56.871) (end 68 54.775) (width 1) (layer "B.Cu") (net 1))
 (segment (start 90.11 63) (end 93 63) (width 1) (layer "B.Cu") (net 10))
 (segment (start 85.5112 58.4012) (end 90.11 63) (width 1) (layer "B.Cu") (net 10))
 (segment (start 78.5 45.5) (end 78.5 46.31) (width 1) (layer "B.Cu") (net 9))
 (segment (start 78.5 46.31) (end 85.5112 53.3212) (width 1) (layer "B.Cu") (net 9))
 (segment (start 80.4312 63.4812) (end 85.5112 63.4812) (width 1) (layer "B.Cu") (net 8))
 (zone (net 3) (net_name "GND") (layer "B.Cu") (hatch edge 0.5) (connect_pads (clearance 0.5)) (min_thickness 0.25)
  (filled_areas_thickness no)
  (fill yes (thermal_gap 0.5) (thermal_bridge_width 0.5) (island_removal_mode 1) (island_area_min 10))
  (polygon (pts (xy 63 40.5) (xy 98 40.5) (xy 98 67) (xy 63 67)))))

